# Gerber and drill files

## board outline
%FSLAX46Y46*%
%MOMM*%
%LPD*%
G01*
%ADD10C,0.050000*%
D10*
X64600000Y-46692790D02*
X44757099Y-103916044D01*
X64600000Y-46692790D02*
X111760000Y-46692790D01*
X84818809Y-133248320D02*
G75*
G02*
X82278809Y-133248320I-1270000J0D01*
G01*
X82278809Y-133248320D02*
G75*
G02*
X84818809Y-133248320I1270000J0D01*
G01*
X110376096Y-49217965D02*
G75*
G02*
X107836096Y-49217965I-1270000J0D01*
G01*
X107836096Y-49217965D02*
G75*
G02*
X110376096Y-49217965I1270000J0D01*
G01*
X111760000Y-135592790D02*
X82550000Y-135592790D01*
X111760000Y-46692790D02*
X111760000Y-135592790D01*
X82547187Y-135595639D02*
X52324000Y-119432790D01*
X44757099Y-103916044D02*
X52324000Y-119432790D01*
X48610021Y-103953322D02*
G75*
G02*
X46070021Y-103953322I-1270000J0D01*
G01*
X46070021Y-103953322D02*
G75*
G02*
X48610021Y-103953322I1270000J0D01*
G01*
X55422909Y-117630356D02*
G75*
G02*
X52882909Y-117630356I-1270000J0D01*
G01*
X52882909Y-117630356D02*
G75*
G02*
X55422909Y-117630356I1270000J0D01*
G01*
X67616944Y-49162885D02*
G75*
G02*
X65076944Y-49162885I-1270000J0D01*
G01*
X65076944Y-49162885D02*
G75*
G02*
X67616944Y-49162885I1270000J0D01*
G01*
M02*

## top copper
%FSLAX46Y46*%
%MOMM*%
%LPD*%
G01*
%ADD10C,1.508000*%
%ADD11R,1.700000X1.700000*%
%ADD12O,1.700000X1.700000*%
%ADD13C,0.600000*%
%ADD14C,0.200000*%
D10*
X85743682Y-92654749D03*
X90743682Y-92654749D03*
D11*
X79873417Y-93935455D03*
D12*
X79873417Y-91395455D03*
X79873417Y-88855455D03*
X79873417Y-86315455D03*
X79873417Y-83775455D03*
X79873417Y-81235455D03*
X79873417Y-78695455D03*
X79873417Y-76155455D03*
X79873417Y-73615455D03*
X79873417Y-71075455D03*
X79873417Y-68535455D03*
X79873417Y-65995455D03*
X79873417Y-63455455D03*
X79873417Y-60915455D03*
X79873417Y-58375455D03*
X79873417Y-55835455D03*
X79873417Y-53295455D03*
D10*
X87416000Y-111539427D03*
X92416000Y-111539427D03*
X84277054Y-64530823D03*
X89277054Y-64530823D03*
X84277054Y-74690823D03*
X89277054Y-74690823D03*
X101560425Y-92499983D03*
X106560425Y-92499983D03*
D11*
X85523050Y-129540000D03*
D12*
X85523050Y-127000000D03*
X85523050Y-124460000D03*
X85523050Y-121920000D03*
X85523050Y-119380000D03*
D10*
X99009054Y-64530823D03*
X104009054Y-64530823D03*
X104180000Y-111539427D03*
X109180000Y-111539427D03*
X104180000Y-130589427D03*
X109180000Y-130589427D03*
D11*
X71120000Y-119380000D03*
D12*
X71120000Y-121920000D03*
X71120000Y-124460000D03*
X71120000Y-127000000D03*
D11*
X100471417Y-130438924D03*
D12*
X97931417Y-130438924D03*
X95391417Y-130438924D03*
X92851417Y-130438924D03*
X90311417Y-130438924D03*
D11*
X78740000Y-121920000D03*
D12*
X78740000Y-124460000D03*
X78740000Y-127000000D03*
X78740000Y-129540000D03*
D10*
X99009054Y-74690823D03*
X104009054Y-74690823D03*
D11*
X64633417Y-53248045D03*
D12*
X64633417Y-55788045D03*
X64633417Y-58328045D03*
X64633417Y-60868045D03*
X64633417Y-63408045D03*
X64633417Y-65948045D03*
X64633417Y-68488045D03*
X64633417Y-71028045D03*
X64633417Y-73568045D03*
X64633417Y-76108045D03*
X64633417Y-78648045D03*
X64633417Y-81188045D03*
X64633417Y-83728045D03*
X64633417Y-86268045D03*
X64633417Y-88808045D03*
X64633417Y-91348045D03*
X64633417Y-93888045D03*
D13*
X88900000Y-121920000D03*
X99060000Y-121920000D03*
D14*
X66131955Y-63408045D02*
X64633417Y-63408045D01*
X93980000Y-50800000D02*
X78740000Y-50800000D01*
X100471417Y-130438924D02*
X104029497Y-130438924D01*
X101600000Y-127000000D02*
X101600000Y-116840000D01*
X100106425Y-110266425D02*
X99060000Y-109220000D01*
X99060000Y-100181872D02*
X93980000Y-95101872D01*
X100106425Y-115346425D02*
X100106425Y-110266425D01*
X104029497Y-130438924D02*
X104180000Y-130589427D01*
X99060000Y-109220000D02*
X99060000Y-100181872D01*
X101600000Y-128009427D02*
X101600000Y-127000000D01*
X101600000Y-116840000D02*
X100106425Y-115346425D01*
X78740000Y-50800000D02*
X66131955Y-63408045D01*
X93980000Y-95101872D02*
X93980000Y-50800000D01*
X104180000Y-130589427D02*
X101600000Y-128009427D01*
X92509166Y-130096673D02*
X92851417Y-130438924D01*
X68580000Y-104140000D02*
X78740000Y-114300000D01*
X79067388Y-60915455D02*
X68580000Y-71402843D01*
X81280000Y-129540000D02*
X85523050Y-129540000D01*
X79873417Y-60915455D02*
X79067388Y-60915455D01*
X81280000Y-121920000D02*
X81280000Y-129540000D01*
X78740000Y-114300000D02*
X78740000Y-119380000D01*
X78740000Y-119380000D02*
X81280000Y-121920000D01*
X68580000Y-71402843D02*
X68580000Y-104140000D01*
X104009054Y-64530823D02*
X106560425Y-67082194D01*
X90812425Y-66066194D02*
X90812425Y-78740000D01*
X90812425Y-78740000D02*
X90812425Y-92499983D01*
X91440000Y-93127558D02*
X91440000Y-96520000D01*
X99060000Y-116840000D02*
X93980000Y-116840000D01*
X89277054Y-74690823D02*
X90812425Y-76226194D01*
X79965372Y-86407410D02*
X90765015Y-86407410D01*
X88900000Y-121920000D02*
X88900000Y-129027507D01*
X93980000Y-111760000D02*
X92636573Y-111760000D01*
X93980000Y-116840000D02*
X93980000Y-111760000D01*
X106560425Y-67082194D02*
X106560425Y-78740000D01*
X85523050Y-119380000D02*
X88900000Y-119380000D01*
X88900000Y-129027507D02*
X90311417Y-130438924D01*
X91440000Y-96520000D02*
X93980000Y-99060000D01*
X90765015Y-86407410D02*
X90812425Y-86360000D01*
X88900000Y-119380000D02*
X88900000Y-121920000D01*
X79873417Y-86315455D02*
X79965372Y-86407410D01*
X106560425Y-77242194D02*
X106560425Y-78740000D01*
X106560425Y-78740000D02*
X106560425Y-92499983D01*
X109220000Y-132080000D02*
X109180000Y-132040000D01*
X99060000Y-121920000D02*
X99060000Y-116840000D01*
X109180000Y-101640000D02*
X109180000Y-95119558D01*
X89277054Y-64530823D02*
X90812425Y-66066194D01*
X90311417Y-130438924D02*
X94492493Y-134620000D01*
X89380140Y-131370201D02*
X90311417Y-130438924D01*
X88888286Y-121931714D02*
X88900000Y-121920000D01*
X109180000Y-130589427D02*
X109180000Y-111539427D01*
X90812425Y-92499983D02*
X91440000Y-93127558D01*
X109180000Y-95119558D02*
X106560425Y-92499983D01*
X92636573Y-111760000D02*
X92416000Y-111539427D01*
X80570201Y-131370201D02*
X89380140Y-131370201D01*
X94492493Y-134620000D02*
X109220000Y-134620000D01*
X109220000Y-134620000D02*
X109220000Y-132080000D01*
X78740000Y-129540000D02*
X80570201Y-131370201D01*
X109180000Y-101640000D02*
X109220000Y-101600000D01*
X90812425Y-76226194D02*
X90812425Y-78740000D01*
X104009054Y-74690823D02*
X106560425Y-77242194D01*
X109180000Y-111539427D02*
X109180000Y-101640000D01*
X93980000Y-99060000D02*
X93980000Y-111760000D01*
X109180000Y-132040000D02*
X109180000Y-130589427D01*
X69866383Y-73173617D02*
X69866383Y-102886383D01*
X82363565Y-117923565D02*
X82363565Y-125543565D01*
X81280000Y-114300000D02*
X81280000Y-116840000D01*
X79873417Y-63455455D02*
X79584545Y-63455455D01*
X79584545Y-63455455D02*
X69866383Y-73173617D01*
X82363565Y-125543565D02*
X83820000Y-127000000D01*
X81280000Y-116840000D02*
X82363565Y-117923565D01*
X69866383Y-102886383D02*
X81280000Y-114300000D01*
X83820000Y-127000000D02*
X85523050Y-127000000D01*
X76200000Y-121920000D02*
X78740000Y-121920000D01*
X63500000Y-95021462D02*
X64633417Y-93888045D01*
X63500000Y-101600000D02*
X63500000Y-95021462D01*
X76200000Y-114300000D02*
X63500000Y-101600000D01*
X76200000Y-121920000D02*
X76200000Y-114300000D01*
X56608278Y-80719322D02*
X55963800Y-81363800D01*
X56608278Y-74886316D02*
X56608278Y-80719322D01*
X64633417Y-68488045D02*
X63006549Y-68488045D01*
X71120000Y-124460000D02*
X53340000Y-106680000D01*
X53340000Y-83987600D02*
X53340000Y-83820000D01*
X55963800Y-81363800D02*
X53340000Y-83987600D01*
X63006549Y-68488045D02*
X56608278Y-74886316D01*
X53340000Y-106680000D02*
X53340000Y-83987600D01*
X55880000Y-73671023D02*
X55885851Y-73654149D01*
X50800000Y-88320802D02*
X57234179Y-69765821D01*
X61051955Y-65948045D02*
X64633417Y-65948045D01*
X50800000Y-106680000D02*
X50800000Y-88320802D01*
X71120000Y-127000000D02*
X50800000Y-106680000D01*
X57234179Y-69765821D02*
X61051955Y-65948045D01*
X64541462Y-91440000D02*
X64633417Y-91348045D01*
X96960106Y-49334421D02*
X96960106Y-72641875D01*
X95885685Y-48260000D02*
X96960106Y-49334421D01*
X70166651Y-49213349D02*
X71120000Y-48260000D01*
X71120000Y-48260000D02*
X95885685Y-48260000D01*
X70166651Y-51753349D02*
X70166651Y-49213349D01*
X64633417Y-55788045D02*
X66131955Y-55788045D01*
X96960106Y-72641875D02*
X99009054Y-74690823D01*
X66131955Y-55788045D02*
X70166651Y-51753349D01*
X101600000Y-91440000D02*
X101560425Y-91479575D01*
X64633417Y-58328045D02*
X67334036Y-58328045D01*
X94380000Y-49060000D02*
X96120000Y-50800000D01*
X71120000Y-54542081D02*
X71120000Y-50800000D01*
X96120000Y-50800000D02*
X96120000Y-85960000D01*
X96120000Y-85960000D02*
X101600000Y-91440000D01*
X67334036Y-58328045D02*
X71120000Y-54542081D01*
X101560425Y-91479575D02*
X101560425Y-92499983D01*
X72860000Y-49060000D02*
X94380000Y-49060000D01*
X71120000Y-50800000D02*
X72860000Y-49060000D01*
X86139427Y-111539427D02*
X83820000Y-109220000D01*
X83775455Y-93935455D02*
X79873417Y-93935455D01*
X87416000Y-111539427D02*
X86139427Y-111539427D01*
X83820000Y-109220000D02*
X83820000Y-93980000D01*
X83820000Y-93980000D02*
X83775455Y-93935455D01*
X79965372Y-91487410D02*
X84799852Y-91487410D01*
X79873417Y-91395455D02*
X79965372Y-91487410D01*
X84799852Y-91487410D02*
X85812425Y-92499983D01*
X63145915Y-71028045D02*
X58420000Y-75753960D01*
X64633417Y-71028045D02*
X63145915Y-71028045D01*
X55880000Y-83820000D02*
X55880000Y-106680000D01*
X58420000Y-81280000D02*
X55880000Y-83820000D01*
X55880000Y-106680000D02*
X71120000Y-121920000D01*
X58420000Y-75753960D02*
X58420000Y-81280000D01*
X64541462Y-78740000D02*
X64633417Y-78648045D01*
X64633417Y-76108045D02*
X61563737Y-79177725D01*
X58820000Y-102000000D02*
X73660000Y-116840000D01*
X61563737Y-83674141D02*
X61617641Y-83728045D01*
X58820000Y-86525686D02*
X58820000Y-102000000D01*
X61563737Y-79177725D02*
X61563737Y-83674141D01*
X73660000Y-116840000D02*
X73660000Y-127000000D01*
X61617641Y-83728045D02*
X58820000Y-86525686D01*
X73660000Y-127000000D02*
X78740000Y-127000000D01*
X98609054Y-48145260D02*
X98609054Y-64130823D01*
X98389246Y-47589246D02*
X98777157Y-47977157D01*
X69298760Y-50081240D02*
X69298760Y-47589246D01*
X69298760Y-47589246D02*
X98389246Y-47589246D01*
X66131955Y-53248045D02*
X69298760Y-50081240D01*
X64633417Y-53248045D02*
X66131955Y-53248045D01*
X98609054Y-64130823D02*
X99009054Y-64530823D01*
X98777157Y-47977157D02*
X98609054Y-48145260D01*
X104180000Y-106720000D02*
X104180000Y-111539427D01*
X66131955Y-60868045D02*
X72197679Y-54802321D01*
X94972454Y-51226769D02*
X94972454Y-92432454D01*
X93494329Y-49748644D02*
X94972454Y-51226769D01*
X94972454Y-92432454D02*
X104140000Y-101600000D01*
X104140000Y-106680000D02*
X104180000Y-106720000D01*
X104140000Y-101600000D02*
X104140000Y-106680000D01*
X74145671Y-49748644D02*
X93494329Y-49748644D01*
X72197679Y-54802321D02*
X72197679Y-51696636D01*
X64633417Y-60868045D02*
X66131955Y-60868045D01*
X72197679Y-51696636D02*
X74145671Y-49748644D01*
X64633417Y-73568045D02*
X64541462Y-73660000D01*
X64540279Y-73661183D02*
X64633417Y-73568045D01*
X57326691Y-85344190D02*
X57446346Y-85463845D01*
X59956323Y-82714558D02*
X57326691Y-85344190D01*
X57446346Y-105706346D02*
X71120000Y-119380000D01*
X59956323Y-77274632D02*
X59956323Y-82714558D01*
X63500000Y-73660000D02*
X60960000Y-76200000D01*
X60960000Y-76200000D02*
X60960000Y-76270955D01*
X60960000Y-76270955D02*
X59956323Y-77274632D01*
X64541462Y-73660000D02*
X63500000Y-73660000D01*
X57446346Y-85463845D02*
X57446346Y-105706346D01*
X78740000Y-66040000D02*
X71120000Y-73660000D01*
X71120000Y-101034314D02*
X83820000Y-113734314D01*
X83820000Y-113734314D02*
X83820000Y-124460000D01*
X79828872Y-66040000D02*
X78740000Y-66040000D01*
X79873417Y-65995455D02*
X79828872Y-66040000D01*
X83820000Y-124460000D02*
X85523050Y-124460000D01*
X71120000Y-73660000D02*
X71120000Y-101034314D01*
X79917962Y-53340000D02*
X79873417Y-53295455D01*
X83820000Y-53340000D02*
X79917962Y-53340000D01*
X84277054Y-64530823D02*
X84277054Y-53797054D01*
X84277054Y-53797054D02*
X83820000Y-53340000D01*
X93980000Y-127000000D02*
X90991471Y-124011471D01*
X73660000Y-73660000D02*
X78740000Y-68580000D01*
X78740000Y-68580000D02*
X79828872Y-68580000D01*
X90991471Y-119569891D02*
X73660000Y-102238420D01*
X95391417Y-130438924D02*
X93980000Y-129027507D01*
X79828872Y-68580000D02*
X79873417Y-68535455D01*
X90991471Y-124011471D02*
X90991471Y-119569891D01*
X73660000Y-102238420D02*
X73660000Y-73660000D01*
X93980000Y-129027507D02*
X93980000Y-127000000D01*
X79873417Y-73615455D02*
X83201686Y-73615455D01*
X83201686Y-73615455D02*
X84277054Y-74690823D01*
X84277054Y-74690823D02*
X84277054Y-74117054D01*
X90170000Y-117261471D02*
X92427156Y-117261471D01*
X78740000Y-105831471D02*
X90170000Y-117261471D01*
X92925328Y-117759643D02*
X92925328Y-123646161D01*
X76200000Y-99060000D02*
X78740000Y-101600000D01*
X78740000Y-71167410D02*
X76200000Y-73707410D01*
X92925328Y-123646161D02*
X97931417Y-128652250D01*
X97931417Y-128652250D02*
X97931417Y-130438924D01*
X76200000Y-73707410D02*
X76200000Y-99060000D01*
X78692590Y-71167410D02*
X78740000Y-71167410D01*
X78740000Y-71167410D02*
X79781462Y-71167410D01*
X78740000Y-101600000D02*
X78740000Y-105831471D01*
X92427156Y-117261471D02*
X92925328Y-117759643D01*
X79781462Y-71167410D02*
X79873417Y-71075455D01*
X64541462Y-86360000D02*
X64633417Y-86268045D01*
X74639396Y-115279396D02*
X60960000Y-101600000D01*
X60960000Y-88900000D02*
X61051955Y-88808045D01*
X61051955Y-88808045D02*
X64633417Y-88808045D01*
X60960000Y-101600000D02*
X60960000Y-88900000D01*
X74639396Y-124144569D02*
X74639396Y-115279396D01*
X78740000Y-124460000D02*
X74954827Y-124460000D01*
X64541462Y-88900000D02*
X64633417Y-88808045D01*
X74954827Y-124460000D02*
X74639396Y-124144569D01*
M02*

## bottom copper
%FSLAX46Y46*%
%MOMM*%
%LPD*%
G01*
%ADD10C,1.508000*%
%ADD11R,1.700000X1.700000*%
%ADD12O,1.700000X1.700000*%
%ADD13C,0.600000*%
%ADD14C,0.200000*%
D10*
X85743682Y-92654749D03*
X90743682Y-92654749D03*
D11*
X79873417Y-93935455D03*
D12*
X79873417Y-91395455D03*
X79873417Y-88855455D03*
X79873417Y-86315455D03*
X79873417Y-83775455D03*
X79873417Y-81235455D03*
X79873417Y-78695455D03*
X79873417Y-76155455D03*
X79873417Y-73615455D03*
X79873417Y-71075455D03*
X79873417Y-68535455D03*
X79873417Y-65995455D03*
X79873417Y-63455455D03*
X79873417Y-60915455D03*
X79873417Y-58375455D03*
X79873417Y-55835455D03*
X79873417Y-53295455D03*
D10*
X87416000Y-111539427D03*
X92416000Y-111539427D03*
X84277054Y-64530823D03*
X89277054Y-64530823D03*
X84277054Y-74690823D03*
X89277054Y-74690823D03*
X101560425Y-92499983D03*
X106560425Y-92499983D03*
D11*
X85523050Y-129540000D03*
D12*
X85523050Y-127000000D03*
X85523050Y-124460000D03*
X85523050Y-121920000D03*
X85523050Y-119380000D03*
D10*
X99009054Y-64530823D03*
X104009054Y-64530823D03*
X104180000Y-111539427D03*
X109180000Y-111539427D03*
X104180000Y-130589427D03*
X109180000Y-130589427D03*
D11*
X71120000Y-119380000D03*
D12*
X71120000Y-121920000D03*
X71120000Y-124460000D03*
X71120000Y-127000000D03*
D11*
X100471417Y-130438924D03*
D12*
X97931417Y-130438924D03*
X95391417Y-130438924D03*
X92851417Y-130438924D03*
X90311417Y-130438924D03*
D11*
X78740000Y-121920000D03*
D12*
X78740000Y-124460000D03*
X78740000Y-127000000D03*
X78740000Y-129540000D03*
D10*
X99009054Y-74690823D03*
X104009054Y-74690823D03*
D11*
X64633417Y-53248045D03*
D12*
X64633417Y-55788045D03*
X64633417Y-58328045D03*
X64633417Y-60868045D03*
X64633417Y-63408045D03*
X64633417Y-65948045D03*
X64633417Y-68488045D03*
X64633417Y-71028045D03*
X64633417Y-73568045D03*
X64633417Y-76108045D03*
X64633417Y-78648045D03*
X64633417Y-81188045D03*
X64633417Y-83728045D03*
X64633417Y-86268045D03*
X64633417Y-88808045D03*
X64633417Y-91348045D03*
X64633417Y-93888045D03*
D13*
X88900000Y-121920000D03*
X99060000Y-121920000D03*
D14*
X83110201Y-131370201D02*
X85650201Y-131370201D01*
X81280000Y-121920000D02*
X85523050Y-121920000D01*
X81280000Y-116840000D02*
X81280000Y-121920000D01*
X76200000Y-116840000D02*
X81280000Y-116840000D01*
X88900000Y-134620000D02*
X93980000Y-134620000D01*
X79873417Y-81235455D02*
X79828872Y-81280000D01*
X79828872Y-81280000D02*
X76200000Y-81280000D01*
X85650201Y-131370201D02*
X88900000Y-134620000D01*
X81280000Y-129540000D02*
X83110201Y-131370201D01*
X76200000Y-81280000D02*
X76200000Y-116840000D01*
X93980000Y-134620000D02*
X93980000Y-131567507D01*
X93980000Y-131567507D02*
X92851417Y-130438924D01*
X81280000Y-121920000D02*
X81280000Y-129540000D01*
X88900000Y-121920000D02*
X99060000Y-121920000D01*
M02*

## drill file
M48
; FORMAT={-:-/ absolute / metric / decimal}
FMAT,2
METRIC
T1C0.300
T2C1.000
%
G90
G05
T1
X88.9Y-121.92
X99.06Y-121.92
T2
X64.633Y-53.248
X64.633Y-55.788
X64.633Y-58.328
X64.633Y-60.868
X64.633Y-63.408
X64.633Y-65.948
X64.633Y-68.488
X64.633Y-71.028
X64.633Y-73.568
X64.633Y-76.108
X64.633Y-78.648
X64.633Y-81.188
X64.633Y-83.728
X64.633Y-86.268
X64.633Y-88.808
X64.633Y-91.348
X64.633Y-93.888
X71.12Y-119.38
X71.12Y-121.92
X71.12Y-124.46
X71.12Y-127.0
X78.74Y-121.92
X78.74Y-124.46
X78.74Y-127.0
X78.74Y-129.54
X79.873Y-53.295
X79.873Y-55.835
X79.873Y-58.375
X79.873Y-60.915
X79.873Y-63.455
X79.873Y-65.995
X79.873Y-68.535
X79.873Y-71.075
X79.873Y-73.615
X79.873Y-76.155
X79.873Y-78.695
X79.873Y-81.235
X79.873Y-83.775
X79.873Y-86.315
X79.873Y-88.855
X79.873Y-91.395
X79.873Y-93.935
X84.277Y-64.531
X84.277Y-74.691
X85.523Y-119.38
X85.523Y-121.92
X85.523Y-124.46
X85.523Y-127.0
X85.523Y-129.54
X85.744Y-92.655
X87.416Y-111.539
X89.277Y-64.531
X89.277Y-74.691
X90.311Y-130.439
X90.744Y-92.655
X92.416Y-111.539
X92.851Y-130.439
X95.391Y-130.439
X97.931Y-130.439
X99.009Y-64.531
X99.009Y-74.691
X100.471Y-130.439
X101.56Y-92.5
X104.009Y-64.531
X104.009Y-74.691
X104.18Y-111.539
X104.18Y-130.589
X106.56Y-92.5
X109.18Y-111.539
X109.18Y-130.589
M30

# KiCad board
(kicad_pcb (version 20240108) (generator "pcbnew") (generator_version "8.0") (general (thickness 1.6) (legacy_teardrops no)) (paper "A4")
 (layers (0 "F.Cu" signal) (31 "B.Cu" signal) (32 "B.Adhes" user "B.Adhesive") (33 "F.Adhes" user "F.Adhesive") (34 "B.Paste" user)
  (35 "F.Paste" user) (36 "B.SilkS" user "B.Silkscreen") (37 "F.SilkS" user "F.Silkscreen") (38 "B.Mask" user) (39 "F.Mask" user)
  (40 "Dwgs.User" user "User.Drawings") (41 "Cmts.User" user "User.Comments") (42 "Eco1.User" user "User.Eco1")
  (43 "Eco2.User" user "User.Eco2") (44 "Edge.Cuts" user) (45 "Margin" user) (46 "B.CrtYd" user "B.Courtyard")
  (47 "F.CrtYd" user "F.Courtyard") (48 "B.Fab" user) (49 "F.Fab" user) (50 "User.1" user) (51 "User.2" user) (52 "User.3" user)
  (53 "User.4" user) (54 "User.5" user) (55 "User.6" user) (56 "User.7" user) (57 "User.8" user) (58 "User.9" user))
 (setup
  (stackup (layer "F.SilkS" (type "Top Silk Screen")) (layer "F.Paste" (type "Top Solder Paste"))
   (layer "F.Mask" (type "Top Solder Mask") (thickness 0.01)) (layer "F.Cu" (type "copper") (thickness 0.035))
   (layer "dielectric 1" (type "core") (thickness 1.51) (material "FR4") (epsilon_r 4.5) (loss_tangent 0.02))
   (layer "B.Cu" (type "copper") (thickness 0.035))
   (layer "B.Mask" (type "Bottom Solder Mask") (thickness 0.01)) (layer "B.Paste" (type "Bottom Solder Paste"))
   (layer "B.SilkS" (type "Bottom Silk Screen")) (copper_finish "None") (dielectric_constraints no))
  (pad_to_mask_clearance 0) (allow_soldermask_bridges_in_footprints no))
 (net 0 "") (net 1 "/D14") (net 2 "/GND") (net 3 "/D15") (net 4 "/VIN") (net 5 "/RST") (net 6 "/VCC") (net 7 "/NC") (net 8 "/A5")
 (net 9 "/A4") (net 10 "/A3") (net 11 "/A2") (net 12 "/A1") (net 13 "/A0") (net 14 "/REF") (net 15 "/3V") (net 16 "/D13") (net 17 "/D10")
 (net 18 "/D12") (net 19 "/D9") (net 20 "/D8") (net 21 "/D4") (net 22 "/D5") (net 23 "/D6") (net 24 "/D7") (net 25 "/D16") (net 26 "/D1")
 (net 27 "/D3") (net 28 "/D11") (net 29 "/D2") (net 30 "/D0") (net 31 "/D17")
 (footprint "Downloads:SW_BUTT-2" (layer "F.Cu") (at 88.243682 92.654749)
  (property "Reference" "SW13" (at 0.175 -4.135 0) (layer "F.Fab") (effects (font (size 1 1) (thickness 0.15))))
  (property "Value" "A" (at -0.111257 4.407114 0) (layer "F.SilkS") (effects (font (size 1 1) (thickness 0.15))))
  (pad "1" thru_hole circle (at -2.5 0) (size 1.508 1.508) (drill 1) (layers "*.Cu" "*.Mask") (remove_unused_layers no) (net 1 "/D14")
   (solder_mask_margin 0.102))
  (pad "2" thru_hole circle (at 2.5 0) (size 1.508 1.508) (drill 1) (layers "*.Cu" "*.Mask") (remove_unused_layers no) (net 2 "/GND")
   (solder_mask_margin 0.102)))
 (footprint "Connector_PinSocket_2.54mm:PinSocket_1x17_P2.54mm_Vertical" (layer "F.Cu") (at 79.873417 93.935455 180)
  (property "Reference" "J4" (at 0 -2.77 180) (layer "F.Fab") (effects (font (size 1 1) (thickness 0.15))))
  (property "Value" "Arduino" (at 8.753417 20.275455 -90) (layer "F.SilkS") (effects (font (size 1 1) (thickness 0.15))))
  (pad "1" thru_hole rect (at 0 0 180) (size 1.7 1.7) (drill 1) (layers "*.Cu" "*.Mask") (remove_unused_layers no) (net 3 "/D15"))
  (pad "2" thru_hole oval (at 0 2.54 180) (size 1.7 1.7) (drill 1) (layers "*.Cu" "*.Mask") (remove_unused_layers no) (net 1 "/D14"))
  (pad "3" thru_hole oval (at 0 5.08 180) (size 1.7 1.7) (drill 1) (layers "*.Cu" "*.Mask") (remove_unused_layers no) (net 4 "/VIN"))
  (pad "4" thru_hole oval (at 0 7.62 180) (size 1.7 1.7) (drill 1) (layers "*.Cu" "*.Mask") (remove_unused_layers no) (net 2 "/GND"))
  (pad "5" thru_hole oval (at 0 10.16 180) (size 1.7 1.7) (drill 1) (layers "*.Cu" "*.Mask") (remove_unused_layers no) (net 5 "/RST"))
  (pad "6" thru_hole oval (at 0 12.7 180) (size 1.7 1.7) (drill 1) (layers "*.Cu" "*.Mask") (remove_unused_layers no) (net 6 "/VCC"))
  (pad "7" thru_hole oval (at 0 15.24 180) (size 1.7 1.7) (drill 1) (layers "*.Cu" "*.Mask") (remove_unused_layers no) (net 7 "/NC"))
  (pad "8" thru_hole oval (at 0 17.78 180) (size 1.7 1.7) (drill 1) (layers "*.Cu" "*.Mask") (remove_unused_layers no) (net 7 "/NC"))
  (pad "9" thru_hole oval (at 0 20.32 180) (size 1.7 1.7) (drill 1) (layers "*.Cu" "*.Mask") (remove_unused_layers no) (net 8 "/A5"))
  (pad "10" thru_hole oval (at 0 22.86 180) (size 1.7 1.7) (drill 1) (layers "*.Cu" "*.Mask") (remove_unused_layers no) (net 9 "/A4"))
  (pad "11" thru_hole oval (at 0 25.4 180) (size 1.7 1.7) (drill 1) (layers "*.Cu" "*.Mask") (remove_unused_layers no) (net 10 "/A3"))
  (pad "12" thru_hole oval (at 0 27.94 180) (size 1.7 1.7) (drill 1) (layers "*.Cu" "*.Mask") (remove_unused_layers no) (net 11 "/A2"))
  (pad "13" thru_hole oval (at 0 30.48 180) (size 1.7 1.7) (drill 1) (layers "*.Cu" "*.Mask") (remove_unused_layers no) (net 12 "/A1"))
  (pad "14" thru_hole oval (at 0 33.02 180) (size 1.7 1.7) (drill 1) (layers "*.Cu" "*.Mask") (remove_unused_layers no) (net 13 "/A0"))
  (pad "15" thru_hole oval (at 0 35.56 180) (size 1.7 1.7) (drill 1) (layers "*.Cu" "*.Mask") (remove_unused_layers no) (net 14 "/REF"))
  (pad "16" thru_hole oval (at 0 38.1 180) (size 1.7 1.7) (drill 1) (layers "*.Cu" "*.Mask") (remove_unused_layers no) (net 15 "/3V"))
  (pad "17" thru_hole oval (at 0 40.64 180) (size 1.7 1.7) (drill 1) (layers "*.Cu" "*.Mask") (remove_unused_layers no) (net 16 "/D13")))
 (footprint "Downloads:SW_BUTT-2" (layer "F.Cu") (at 89.916 111.539427)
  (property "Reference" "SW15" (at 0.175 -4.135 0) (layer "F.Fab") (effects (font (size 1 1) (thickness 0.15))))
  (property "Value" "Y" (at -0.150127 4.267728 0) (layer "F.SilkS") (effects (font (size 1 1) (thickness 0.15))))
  (pad "1" thru_hole circle (at -2.5 0) (size 1.508 1.508) (drill 1) (layers "*.Cu" "*.Mask") (remove_unused_layers no) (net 3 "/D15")
   (solder_mask_margin 0.102))
  (pad "2" thru_hole circle (at 2.5 0) (size 1.508 1.508) (drill 1) (layers "*.Cu" "*.Mask") (remove_unused_layers no) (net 2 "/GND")
   (solder_mask_margin 0.102)))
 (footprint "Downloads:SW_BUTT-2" (layer "F.Cu") (at 86.777054 64.530823)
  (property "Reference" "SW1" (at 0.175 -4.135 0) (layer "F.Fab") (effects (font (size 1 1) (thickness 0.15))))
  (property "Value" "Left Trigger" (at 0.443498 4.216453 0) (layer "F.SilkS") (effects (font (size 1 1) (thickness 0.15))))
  (pad "1" thru_hole circle (at -2.5 0) (size 1.508 1.508) (drill 1) (layers "*.Cu" "*.Mask") (remove_unused_layers no) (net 16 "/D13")
   (solder_mask_margin 0.102))
  (pad "2" thru_hole circle (at 2.5 0) (size 1.508 1.508) (drill 1) (layers "*.Cu" "*.Mask") (remove_unused_layers no) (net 2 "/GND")
   (solder_mask_margin 0.102)))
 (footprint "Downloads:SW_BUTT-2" (layer "F.Cu") (at 86.777054 74.690823)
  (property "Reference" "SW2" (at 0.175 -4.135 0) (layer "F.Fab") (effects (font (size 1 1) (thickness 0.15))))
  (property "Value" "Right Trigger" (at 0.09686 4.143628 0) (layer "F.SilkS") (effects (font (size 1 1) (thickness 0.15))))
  (pad "1" thru_hole circle (at -2.5 0) (size 1.508 1.508) (drill 1) (layers "*.Cu" "*.Mask") (remove_unused_layers no) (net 8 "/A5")
   (solder_mask_margin 0.102))
  (pad "2" thru_hole circle (at 2.5 0) (size 1.508 1.508) (drill 1) (layers "*.Cu" "*.Mask") (remove_unused_layers no) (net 2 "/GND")
   (solder_mask_margin 0.102)))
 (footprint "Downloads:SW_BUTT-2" (layer "F.Cu") (at 104.060425 92.499983)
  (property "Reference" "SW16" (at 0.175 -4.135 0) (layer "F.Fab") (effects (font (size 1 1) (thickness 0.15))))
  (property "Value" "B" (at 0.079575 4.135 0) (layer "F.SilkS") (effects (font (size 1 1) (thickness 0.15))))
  (pad "1" thru_hole circle (at -2.5 0) (size 1.508 1.508) (drill 1) (layers "*.Cu" "*.Mask") (remove_unused_layers no) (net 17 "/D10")
   (solder_mask_margin 0.102))
  (pad "2" thru_hole circle (at 2.5 0) (size 1.508 1.508) (drill 1) (layers "*.Cu" "*.Mask") (remove_unused_layers no) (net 2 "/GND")
   (solder_mask_margin 0.102)))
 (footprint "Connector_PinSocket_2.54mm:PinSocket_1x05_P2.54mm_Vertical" (layer "F.Cu") (at 85.52305 129.54 180)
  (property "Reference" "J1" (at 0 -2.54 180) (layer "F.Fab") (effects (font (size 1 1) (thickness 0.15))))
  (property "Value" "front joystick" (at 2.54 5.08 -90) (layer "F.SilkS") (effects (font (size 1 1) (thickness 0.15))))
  (pad "1" thru_hole rect (at 0 0 180) (size 1.7 1.7) (drill 1) (layers "*.Cu" "*.Mask") (remove_unused_layers no) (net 13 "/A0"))
  (pad "2" thru_hole oval (at 0 2.54 180) (size 1.7 1.7) (drill 1) (layers "*.Cu" "*.Mask") (remove_unused_layers no) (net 12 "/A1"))
  (pad "3" thru_hole oval (at 0 5.08 180) (size 1.7 1.7) (drill 1) (layers "*.Cu" "*.Mask") (remove_unused_layers no) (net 11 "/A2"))
  (pad "4" thru_hole oval (at 0 7.62 180) (size 1.7 1.7) (drill 1) (layers "*.Cu" "*.Mask") (remove_unused_layers no) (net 6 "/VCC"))
  (pad "5" thru_hole oval (at 0 10.16 180) (size 1.7 1.7) (drill 1) (layers "*.Cu" "*.Mask") (remove_unused_layers no) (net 2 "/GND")))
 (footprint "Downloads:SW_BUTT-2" (layer "F.Cu") (at 101.509054 64.530823)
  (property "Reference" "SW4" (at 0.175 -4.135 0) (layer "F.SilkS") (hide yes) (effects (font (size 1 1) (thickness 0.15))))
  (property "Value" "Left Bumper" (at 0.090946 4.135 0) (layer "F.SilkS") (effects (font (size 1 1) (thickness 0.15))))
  (pad "1" thru_hole circle (at -2.5 0) (size 1.508 1.508) (drill 1) (layers "*.Cu" "*.Mask") (remove_unused_layers no) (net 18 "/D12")
   (solder_mask_margin 0.102))
  (pad "2" thru_hole circle (at 2.5 0) (size 1.508 1.508) (drill 1) (layers "*.Cu" "*.Mask") (remove_unused_layers no) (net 2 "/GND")
   (solder_mask_margin 0.102)))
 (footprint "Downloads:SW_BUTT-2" (layer "F.Cu") (at 106.68 111.539427)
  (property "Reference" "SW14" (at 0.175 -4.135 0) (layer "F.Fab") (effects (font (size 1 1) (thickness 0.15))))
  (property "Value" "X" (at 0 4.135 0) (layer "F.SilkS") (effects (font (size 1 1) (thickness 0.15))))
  (pad "1" thru_hole circle (at -2.5 0) (size 1.508 1.508) (drill 1) (layers "*.Cu" "*.Mask") (remove_unused_layers no) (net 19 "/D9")
   (solder_mask_margin 0.102))
  (pad "2" thru_hole circle (at 2.5 0) (size 1.508 1.508) (drill 1) (layers "*.Cu" "*.Mask") (remove_unused_layers no) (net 2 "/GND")
   (solder_mask_margin 0.102)))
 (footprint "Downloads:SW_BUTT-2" (layer "F.Cu") (at 106.68 130.589427)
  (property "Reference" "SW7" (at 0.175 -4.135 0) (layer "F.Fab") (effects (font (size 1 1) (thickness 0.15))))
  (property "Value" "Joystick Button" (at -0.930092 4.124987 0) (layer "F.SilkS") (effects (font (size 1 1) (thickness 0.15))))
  (pad "1" thru_hole circle (at -2.5 0) (size 1.508 1.508) (drill 1) (layers "*.Cu" "*.Mask") (remove_unused_layers no) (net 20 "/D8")
   (solder_mask_margin 0.102))
  (pad "2" thru_hole circle (at 2.5 0) (size 1.508 1.508) (drill 1) (layers "*.Cu" "*.Mask") (remove_unused_layers no) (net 2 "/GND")
   (solder_mask_margin 0.102)))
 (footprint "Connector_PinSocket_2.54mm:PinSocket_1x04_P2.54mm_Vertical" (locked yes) (layer "F.Cu") (at 71.12 119.38)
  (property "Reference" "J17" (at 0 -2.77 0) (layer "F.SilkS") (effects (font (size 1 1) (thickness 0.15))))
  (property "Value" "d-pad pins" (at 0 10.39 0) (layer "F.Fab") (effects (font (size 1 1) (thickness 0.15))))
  (pad "1" thru_hole rect (at 0 0) (size 1.7 1.7) (drill 1) (layers "*.Cu" "*.Mask") (remove_unused_layers no) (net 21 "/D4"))
  (pad "2" thru_hole oval (at 0 2.54) (size 1.7 1.7) (drill 1) (layers "*.Cu" "*.Mask") (remove_unused_layers no) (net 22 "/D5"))
  (pad "3" thru_hole oval (at 0 5.08) (size 1.7 1.7) (drill 1) (layers "*.Cu" "*.Mask") (remove_unused_layers no) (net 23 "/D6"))
  (pad "4" thru_hole oval (at 0 7.62) (size 1.7 1.7) (drill 1) (layers "*.Cu" "*.Mask") (remove_unused_layers no) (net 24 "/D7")))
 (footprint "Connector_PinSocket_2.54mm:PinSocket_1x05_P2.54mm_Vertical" (layer "F.Cu") (at 100.471417 130.438924 -90)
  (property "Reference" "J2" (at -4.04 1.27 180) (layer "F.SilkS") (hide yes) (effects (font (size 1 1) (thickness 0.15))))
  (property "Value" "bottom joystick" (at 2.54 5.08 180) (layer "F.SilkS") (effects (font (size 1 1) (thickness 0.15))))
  (pad "1" thru_hole rect (at 0 0 270) (size 1.7 1.7) (drill 1) (layers "*.Cu" "*.Mask") (remove_unused_layers no) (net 20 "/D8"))
  (pad "2" thru_hole oval (at 0 2.54 270) (size 1.7 1.7) (drill 1) (layers "*.Cu" "*.Mask") (remove_unused_layers no) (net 9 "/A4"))
  (pad "3" thru_hole oval (at 0 5.08 270) (size 1.7 1.7) (drill 1) (layers "*.Cu" "*.Mask") (remove_unused_layers no) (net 10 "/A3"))
  (pad "4" thru_hole oval (at 0 7.62 270) (size 1.7 1.7) (drill 1) (layers "*.Cu" "*.Mask") (remove_unused_layers no) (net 6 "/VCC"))
  (pad "5" thru_hole oval (at 0 10.16 270) (size 1.7 1.7) (drill 1) (layers "*.Cu" "*.Mask") (remove_unused_layers no) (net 2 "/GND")))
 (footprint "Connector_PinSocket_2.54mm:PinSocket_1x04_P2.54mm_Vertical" (layer "F.Cu") (at 78.74 121.92)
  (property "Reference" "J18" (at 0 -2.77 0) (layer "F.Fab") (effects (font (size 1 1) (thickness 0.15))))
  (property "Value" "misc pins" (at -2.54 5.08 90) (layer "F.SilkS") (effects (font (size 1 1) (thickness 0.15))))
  (pad "1" thru_hole rect (at 0 0) (size 1.7 1.7) (drill 1) (layers "*.Cu" "*.Mask") (remove_unused_layers no) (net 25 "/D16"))
  (pad "2" thru_hole oval (at 0 2.54) (size 1.7 1.7) (drill 1) (layers "*.Cu" "*.Mask") (remove_unused_layers no) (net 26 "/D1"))
  (pad "3" thru_hole oval (at 0 5.08) (size 1.7 1.7) (drill 1) (layers "*.Cu" "*.Mask") (remove_unused_layers no) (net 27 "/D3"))
  (pad "4" thru_hole oval (at 0 7.62) (size 1.7 1.7) (drill 1) (layers "*.Cu" "*.Mask") (remove_unused_layers no) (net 2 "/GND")))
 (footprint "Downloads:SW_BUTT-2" (layer "F.Cu") (at 101.509054 74.690823)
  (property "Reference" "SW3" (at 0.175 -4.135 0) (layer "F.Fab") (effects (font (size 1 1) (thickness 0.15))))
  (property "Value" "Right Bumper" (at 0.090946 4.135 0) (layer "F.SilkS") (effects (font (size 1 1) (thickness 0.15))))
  (pad "1" thru_hole circle (at -2.5 0) (size 1.508 1.508) (drill 1) (layers "*.Cu" "*.Mask") (remove_unused_layers no) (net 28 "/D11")
   (solder_mask_margin 0.102))
  (pad "2" thru_hole circle (at 2.5 0) (size 1.508 1.508) (drill 1) (layers "*.Cu" "*.Mask") (remove_unused_layers no) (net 2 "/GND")
   (solder_mask_margin 0.102)))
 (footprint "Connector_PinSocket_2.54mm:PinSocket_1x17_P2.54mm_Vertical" (layer "F.Cu") (at 64.633417 53.248045)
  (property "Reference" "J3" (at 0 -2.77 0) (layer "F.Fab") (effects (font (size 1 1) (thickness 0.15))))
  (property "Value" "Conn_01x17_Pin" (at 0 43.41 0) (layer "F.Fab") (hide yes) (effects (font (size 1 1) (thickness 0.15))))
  (pad "1" thru_hole rect (at 0 0) (size 1.7 1.7) (drill 1) (layers "*.Cu" "*.Mask") (remove_unused_layers no) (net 18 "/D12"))
  (pad "2" thru_hole oval (at 0 2.54) (size 1.7 1.7) (drill 1) (layers "*.Cu" "*.Mask") (remove_unused_layers no) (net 28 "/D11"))
  (pad "3" thru_hole oval (at 0 5.08) (size 1.7 1.7) (drill 1) (layers "*.Cu" "*.Mask") (remove_unused_layers no) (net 17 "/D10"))
  (pad "4" thru_hole oval (at 0 7.62) (size 1.7 1.7) (drill 1) (layers "*.Cu" "*.Mask") (remove_unused_layers no) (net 19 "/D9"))
  (pad "5" thru_hole oval (at 0 10.16) (size 1.7 1.7) (drill 1) (layers "*.Cu" "*.Mask") (remove_unused_layers no) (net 20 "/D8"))
  (pad "6" thru_hole oval (at 0 12.7) (size 1.7 1.7) (drill 1) (layers "*.Cu" "*.Mask") (remove_unused_layers no) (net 24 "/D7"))
  (pad "7" thru_hole oval (at 0 15.24) (size 1.7 1.7) (drill 1) (layers "*.Cu" "*.Mask") (remove_unused_layers no) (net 23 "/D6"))
  (pad "8" thru_hole oval (at 0 17.78) (size 1.7 1.7) (drill 1) (layers "*.Cu" "*.Mask") (remove_unused_layers no) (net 22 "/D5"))
  (pad "9" thru_hole oval (at 0 20.32) (size 1.7 1.7) (drill 1) (layers "*.Cu" "*.Mask") (remove_unused_layers no) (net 21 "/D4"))
  (pad "10" thru_hole oval (at 0 22.86) (size 1.7 1.7) (drill 1) (layers "*.Cu" "*.Mask") (remove_unused_layers no) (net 27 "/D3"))
  (pad "11" thru_hole oval (at 0 25.4) (size 1.7 1.7) (drill 1) (layers "*.Cu" "*.Mask") (remove_unused_layers no) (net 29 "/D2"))
  (pad "12" thru_hole oval (at 0 27.94) (size 1.7 1.7) (drill 1) (layers "*.Cu" "*.Mask") (remove_unused_layers no) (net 2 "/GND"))
  (pad "13" thru_hole oval (at 0 30.48) (size 1.7 1.7) (drill 1) (layers "*.Cu" "*.Mask") (remove_unused_layers no) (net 5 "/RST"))
  (pad "14" thru_hole oval (at 0 33.02) (size 1.7 1.7) (drill 1) (layers "*.Cu" "*.Mask") (remove_unused_layers no) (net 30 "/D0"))
  (pad "15" thru_hole oval (at 0 35.56) (size 1.7 1.7) (drill 1) (layers "*.Cu" "*.Mask") (remove_unused_layers no) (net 26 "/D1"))
  (pad "16" thru_hole oval (at 0 38.1) (size 1.7 1.7) (drill 1) (layers "*.Cu" "*.Mask") (remove_unused_layers no) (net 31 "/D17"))
  (pad "17" thru_hole oval (at 0 40.64) (size 1.7 1.7) (drill 1) (layers "*.Cu" "*.Mask") (remove_unused_layers no) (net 25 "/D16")))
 (gr_line (start 64.6 46.69279) (end 44.757099 103.916044) (stroke (width 0.05) (type default)) (layer "Edge.Cuts"))
 (gr_line (start 64.6 46.69279) (end 111.76 46.69279) (stroke (width 0.05) (type default)) (layer "Edge.Cuts"))
 (gr_circle (center 83.548809 133.24832) (end 82.278809 133.24832) (stroke (width 0.05) (type default)) (fill none) (layer "Edge.Cuts"))
 (gr_circle (center 109.106096 49.217965) (end 110.376096 49.217965) (stroke (width 0.05) (type default)) (fill none) (layer "Edge.Cuts"))
 (gr_line (start 111.76 135.59279) (end 82.55 135.59279) (stroke (width 0.05) (type default)) (layer "Edge.Cuts"))
 (gr_line (start 111.76 46.69279) (end 111.76 135.59279) (stroke (width 0.05) (type default)) (layer "Edge.Cuts"))
 (gr_line (start 82.547187 135.595639) (end 52.324 119.43279) (stroke (width 0.05) (type default)) (layer "Edge.Cuts"))
 (gr_line (start 44.757099 103.916044) (end 52.324 119.43279) (stroke (width 0.05) (type default)) (layer "Edge.Cuts"))
 (gr_circle (center 47.340021 103.953322) (end 46.070021 103.953322) (stroke (width 0.05) (type default)) (fill none) (layer "Edge.Cuts"))
 (gr_circle (center 54.152909 117.630356) (end 52.882909 117.630356) (stroke (width 0.05) (type default)) (fill none) (layer "Edge.Cuts"))
 (gr_circle (center 66.346944 49.162885) (end 66.346944 47.892885) (stroke (width 0.05) (type default)) (fill none) (layer "Edge.Cuts"))
 (segment (start 66.131955 63.408045) (end 64.633417 63.408045) (width 0.2) (layer "F.Cu") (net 20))
 (segment (start 93.98 50.8) (end 78.74 50.8) (width 0.2) (layer "F.Cu") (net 20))
 (segment (start 100.471417 130.438924) (end 104.029497 130.438924) (width 0.2) (layer "F.Cu") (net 20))
 (segment (start 101.6 127) (end 101.6 116.84) (width 0.2) (layer "F.Cu") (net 20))
 (segment (start 100.106425 110.266425) (end 99.06 109.22) (width 0.2) (layer "F.Cu") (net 20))
 (segment (start 99.06 100.181872) (end 93.98 95.101872) (width 0.2) (layer "F.Cu") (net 20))
 (segment (start 100.106425 115.346425) (end 100.106425 110.266425) (width 0.2) (layer "F.Cu") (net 20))
 (segment (start 104.029497 130.438924) (end 104.18 130.589427) (width 0.2) (layer "F.Cu") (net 20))
 (segment (start 99.06 109.22) (end 99.06 100.181872) (width 0.2) (layer "F.Cu") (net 20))
 (segment (start 101.6 128.009427) (end 101.6 127) (width 0.2) (layer "F.Cu") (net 20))
 (segment (start 101.6 116.84) (end 100.106425 115.346425) (width 0.2) (layer "F.Cu") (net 20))
 (segment (start 78.74 50.8) (end 66.131955 63.408045) (width 0.2) (layer "F.Cu") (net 20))
 (segment (start 93.98 95.101872) (end 93.98 50.8) (width 0.2) (layer "F.Cu") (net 20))
 (segment (start 104.18 130.589427) (end 101.6 128.009427) (width 0.2) (layer "F.Cu") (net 20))
 (segment (start 92.509166 130.096673) (end 92.851417 130.438924) (width 0.2) (layer "F.Cu") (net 6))
 (segment (start 83.110201 131.370201) (end 85.650201 131.370201) (width 0.2) (layer "B.Cu") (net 6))
 (segment (start 81.28 121.92) (end 85.52305 121.92) (width 0.2) (layer "B.Cu") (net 6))
 (segment (start 81.28 116.84) (end 81.28 121.92) (width 0.2) (layer "B.Cu") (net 6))
 (segment (start 76.2 116.84) (end 81.28 116.84) (width 0.2) (layer "B.Cu") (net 6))
 (segment (start 88.9 134.62) (end 93.98 134.62) (width 0.2) (layer "B.Cu") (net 6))
 (segment (start 79.873417 81.235455) (end 79.828872 81.28) (width 0.2) (layer "B.Cu") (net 6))
 (segment (start 79.828872 81.28) (end 76.2 81.28) (width 0.2) (layer "B.Cu") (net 6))
 (segment (start 85.650201 131.370201) (end 88.9 134.62) (width 0.2) (layer "B.Cu") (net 6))
 (segment (start 81.28 129.54) (end 83.110201 131.370201) (width 0.2) (layer "B.Cu") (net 6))
 (segment (start 76.2 81.28) (end 76.2 116.84) (width 0.2) (layer "B.Cu") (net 6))
 (segment (start 93.98 134.62) (end 93.98 131.567507) (width 0.2) (layer "B.Cu") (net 6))
 (segment (start 93.98 131.567507) (end 92.851417 130.438924) (width 0.2) (layer "B.Cu") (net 6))
 (segment (start 81.28 121.92) (end 81.28 129.54) (width 0.2) (layer "B.Cu") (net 6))
 (segment (start 68.58 104.14) (end 78.74 114.3) (width 0.2) (layer "F.Cu") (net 13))
 (segment (start 79.067388 60.915455) (end 68.58 71.402843) (width 0.2) (layer "F.Cu") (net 13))
 (segment (start 81.28 129.54) (end 85.52305 129.54) (width 0.2) (layer "F.Cu") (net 13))
 (segment (start 79.873417 60.915455) (end 79.067388 60.915455) (width 0.2) (layer "F.Cu") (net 13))
 (segment (start 81.28 121.92) (end 81.28 129.54) (width 0.2) (layer "F.Cu") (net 13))
 (segment (start 78.74 114.3) (end 78.74 119.38) (width 0.2) (layer "F.Cu") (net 13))
 (segment (start 78.74 119.38) (end 81.28 121.92) (width 0.2) (layer "F.Cu") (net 13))
 (segment (start 68.58 71.402843) (end 68.58 104.14) (width 0.2) (layer "F.Cu") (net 13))
 (segment (start 104.009054 64.530823) (end 106.560425 67.082194) (width 0.2) (layer "F.Cu") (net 2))
 (segment (start 90.812425 66.066194) (end 90.812425 78.74) (width 0.2) (layer "F.Cu") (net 2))
 (segment (start 90.812425 78.74) (end 90.812425 92.499983) (width 0.2) (layer "F.Cu") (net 2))
 (segment (start 91.44 93.127558) (end 91.44 96.52) (width 0.2) (layer "F.Cu") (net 2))
 (segment (start 99.06 116.84) (end 93.98 116.84) (width 0.2) (layer "F.Cu") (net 2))
 (segment (start 89.277054 74.690823) (end 90.812425 76.226194) (width 0.2) (layer "F.Cu") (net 2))
 (segment (start 79.965372 86.40741) (end 90.765015 86.40741) (width 0.2) (layer "F.Cu") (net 2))
 (segment (start 88.9 121.92) (end 88.9 129.027507) (width 0.2) (layer "F.Cu") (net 2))
 (segment (start 93.98 111.76) (end 92.636573 111.76) (width 0.2) (layer "F.Cu") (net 2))
 (segment (start 93.98 116.84) (end 93.98 111.76) (width 0.2) (layer "F.Cu") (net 2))
 (segment (start 106.560425 67.082194) (end 106.560425 78.74) (width 0.2) (layer "F.Cu") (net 2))
 (segment (start 85.52305 119.38) (end 88.9 119.38) (width 0.2) (layer "F.Cu") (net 2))
 (segment (start 88.9 129.027507) (end 90.311417 130.438924) (width 0.2) (layer "F.Cu") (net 2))
 (segment (start 91.44 96.52) (end 93.98 99.06) (width 0.2) (layer "F.Cu") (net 2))
 (segment (start 90.765015 86.40741) (end 90.812425 86.36) (width 0.2) (layer "F.Cu") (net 2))
 (segment (start 88.9 119.38) (end 88.9 121.92) (width 0.2) (layer "F.Cu") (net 2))
 (segment (start 79.873417 86.315455) (end 79.965372 86.40741) (width 0.2) (layer "F.Cu") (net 2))
 (segment (start 106.560425 77.242194) (end 106.560425 78.74) (width 0.2) (layer "F.Cu") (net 2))
 (segment (start 106.560425 78.74) (end 106.560425 92.499983) (width 0.2) (layer "F.Cu") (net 2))
 (segment (start 109.22 132.08) (end 109.18 132.04) (width 0.2) (layer "F.Cu") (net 2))
 (segment (start 99.06 121.92) (end 99.06 116.84) (width 0.2) (layer "F.Cu") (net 2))
 (segment (start 109.18 101.64) (end 109.18 95.119558) (width 0.2) (layer "F.Cu") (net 2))
 (segment (start 89.277054 64.530823) (end 90.812425 66.066194) (width 0.2) (layer "F.Cu") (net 2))
 (segment (start 90.311417 130.438924) (end 94.492493 134.62) (width 0.2) (layer "F.Cu") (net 2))
 (segment (start 89.38014 131.370201) (end 90.311417 130.438924) (width 0.2) (layer "F.Cu") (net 2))
 (segment (start 88.888286 121.931714) (end 88.9 121.92) (width 0.2) (layer "F.Cu") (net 2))
 (segment (start 109.18 130.589427) (end 109.18 111.539427) (width 0.2) (layer "F.Cu") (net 2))
 (segment (start 90.812425 92.499983) (end 91.44 93.127558) (width 0.2) (layer "F.Cu") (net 2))
 (segment (start 109.18 95.119558) (end 106.560425 92.499983) (width 0.2) (layer "F.Cu") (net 2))
 (segment (start 92.636573 111.76) (end 92.416 111.539427) (width 0.2) (layer "F.Cu") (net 2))
 (segment (start 80.570201 131.370201) (end 89.38014 131.370201) (width 0.2) (layer "F.Cu") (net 2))
 (segment (start 94.492493 134.62) (end 109.22 134.62) (width 0.2) (layer "F.Cu") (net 2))
 (segment (start 109.22 134.62) (end 109.22 132.08) (width 0.2) (layer "F.Cu") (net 2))
 (segment (start 78.74 129.54) (end 80.570201 131.370201) (width 0.2) (layer "F.Cu") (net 2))
 (segment (start 109.18 101.64) (end 109.22 101.6) (width 0.2) (layer "F.Cu") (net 2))
 (segment (start 90.812425 76.226194) (end 90.812425 78.74) (width 0.2) (layer "F.Cu") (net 2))
 (segment (start 104.009054 74.690823) (end 106.560425 77.242194) (width 0.2) (layer "F.Cu") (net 2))
 (segment (start 109.18 111.539427) (end 109.18 101.64) (width 0.2) (layer "F.Cu") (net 2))
 (segment (start 93.98 99.06) (end 93.98 111.76) (width 0.2) (layer "F.Cu") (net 2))
 (segment (start 109.18 132.04) (end 109.18 130.589427) (width 0.2) (layer "F.Cu") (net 2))
 (via (at 88.9 121.92) (size 0.6) (drill 0.3) (layers "F.Cu" "B.Cu") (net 2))
 (via (at 99.06 121.92) (size 0.6) (drill 0.3) (layers "F.Cu" "B.Cu") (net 2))
 (segment (start 88.9 121.92) (end 99.06 121.92) (width 0.2) (layer "B.Cu") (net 2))
 (segment (start 69.866383 73.173617) (end 69.866383 102.886383) (width 0.2) (layer "F.Cu") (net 12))
 (segment (start 82.363565 117.923565) (end 82.363565 125.543565) (width 0.2) (layer "F.Cu") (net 12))
 (segment (start 81.28 114.3) (end 81.28 116.84) (width 0.2) (layer "F.Cu") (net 12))
 (segment (start 79.873417 63.455455) (end 79.584545 63.455455) (width 0.2) (layer "F.Cu") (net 12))
 (segment (start 79.584545 63.455455) (end 69.866383 73.173617) (width 0.2) (layer "F.Cu") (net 12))
 (segment (start 82.363565 125.543565) (end 83.82 127) (width 0.2) (layer "F.Cu") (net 12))
 (segment (start 81.28 116.84) (end 82.363565 117.923565) (width 0.2) (layer "F.Cu") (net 12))
 (segment (start 69.866383 102.886383) (end 81.28 114.3) (width 0.2) (layer "F.Cu") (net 12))
 (segment (start 83.82 127) (end 85.52305 127) (width 0.2) (layer "F.Cu") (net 12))
 (segment (start 76.2 121.92) (end 78.74 121.92) (width 0.2) (layer "F.Cu") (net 25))
 (segment (start 63.5 95.021462) (end 64.633417 93.888045) (width 0.2) (layer "F.Cu") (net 25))
 (segment (start 63.5 101.6) (end 63.5 95.021462) (width 0.2) (layer "F.Cu") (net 25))
 (segment (start 76.2 114.3) (end 63.5 101.6) (width 0.2) (layer "F.Cu") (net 25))
 (segment (start 76.2 121.92) (end 76.2 114.3) (width 0.2) (layer "F.Cu") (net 25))
 (segment (start 56.608278 80.719322) (end 55.9638 81.3638) (width 0.2) (layer "F.Cu") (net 23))
 (segment (start 56.608278 74.886316) (end 56.608278 80.719322) (width 0.2) (layer "F.Cu") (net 23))
 (segment (start 64.633417 68.488045) (end 63.006549 68.488045) (width 0.2) (layer "F.Cu") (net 23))
 (segment (start 71.12 124.46) (end 53.34 106.68) (width 0.2) (layer "F.Cu") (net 23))
 (segment (start 53.34 83.9876) (end 53.34 83.82) (width 0.2) (layer "F.Cu") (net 23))
 (segment (start 55.9638 81.3638) (end 53.34 83.9876) (width 0.2) (layer "F.Cu") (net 23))
 (segment (start 63.006549 68.488045) (end 56.608278 74.886316) (width 0.2) (layer "F.Cu") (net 23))
 (segment (start 53.34 106.68) (end 53.34 83.9876) (width 0.2) (layer "F.Cu") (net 23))
 (segment (start 55.88 73.671023) (end 55.885851 73.654149) (width 0.2) (layer "F.Cu") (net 24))
 (segment (start 50.8 88.320802) (end 57.234179 69.765821) (width 0.2) (layer "F.Cu") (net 24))
 (segment (start 61.051955 65.948045) (end 64.633417 65.948045) (width 0.2) (layer "F.Cu") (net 24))
 (segment (start 50.8 106.68) (end 50.8 88.320802) (width 0.2) (layer "F.Cu") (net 24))
 (segment (start 71.12 127) (end 50.8 106.68) (width 0.2) (layer "F.Cu") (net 24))
 (segment (start 57.234179 69.765821) (end 61.051955 65.948045) (width 0.2) (layer "F.Cu") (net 24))
 (segment (start 64.541462 91.44) (end 64.633417 91.348045) (width 0.2) (layer "F.Cu") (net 31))
 (segment (start 96.960106 49.334421) (end 96.960106 72.641875) (width 0.2) (layer "F.Cu") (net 28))
 (segment (start 95.885685 48.26) (end 96.960106 49.334421) (width 0.2) (layer "F.Cu") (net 28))
 (segment (start 70.166651 49.213349) (end 71.12 48.26) (width 0.2) (layer "F.Cu") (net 28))
 (segment (start 71.12 48.26) (end 95.885685 48.26) (width 0.2) (layer "F.Cu") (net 28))
 (segment (start 70.166651 51.753349) (end 70.166651 49.213349) (width 0.2) (layer "F.Cu") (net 28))
 (segment (start 64.633417 55.788045) (end 66.131955 55.788045) (width 0.2) (layer "F.Cu") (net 28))
 (segment (start 96.960106 72.641875) (end 99.009054 74.690823) (width 0.2) (layer "F.Cu") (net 28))
 (segment (start 66.131955 55.788045) (end 70.166651 51.753349) (width 0.2) (layer "F.Cu") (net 28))
 (segment (start 101.6 91.44) (end 101.560425 91.479575) (width 0.2) (layer "F.Cu") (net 17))
 (segment (start 64.633417 58.328045) (end 67.334036 58.328045) (width 0.2) (layer "F.Cu") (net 17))
 (segment (start 94.38 49.06) (end 96.12 50.8) (width 0.2) (layer "F.Cu") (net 17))
 (segment (start 71.12 54.542081) (end 71.12 50.8) (width 0.2) (layer "F.Cu") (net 17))
 (segment (start 96.12 50.8) (end 96.12 85.96) (width 0.2) (layer "F.Cu") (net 17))
 (segment (start 96.12 85.96) (end 101.6 91.44) (width 0.2) (layer "F.Cu") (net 17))
 (segment (start 67.334036 58.328045) (end 71.12 54.542081) (width 0.2) (layer "F.Cu") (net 17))
 (segment (start 101.560425 91.479575) (end 101.560425 92.499983) (width 0.2) (layer "F.Cu") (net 17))
 (segment (start 72.86 49.06) (end 94.38 49.06) (width 0.2) (layer "F.Cu") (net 17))
 (segment (start 71.12 50.8) (end 72.86 49.06) (width 0.2) (layer "F.Cu") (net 17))
 (segment (start 86.139427 111.539427) (end 83.82 109.22) (width 0.2) (layer "F.Cu") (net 3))
 (segment (start 83.775455 93.935455) (end 79.873417 93.935455) (width 0.2) (layer "F.Cu") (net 3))
 (segment (start 87.416 111.539427) (end 86.139427 111.539427) (width 0.2) (layer "F.Cu") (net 3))
 (segment (start 83.82 109.22) (end 83.82 93.98) (width 0.2) (layer "F.Cu") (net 3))
 (segment (start 83.82 93.98) (end 83.775455 93.935455) (width 0.2) (layer "F.Cu") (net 3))
 (segment (start 79.965372 91.48741) (end 84.799852 91.48741) (width 0.2) (layer "F.Cu") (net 1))
 (segment (start 79.873417 91.395455) (end 79.965372 91.48741) (width 0.2) (layer "F.Cu") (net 1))
 (segment (start 84.799852 91.48741) (end 85.812425 92.499983) (width 0.2) (layer "F.Cu") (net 1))
 (segment (start 63.145915 71.028045) (end 58.42 75.75396) (width 0.2) (layer "F.Cu") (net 22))
 (segment (start 64.633417 71.028045) (end 63.145915 71.028045) (width 0.2) (layer "F.Cu") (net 22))
 (segment (start 55.88 83.82) (end 55.88 106.68) (width 0.2) (layer "F.Cu") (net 22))
 (segment (start 58.42 81.28) (end 55.88 83.82) (width 0.2) (layer "F.Cu") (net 22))
 (segment (start 55.88 106.68) (end 71.12 121.92) (width 0.2) (layer "F.Cu") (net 22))
 (segment (start 58.42 75.75396) (end 58.42 81.28) (width 0.2) (layer "F.Cu") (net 22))
 (segment (start 64.541462 78.74) (end 64.633417 78.648045) (width 0.2) (layer "F.Cu") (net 29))
 (segment (start 64.633417 76.108045) (end 61.563737 79.177725) (width 0.2) (layer "F.Cu") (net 27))
 (segment (start 58.82 102) (end 73.66 116.84) (width 0.2) (layer "F.Cu") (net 27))
 (segment (start 61.563737 83.674141) (end 61.617641 83.728045) (width 0.2) (layer "F.Cu") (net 27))
 (segment (start 58.82 86.525686) (end 58.82 102) (width 0.2) (layer "F.Cu") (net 27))
 (segment (start 61.563737 79.177725) (end 61.563737 83.674141) (width 0.2) (layer "F.Cu") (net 27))
 (segment (start 73.66 116.84) (end 73.66 127) (width 0.2) (layer "F.Cu") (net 27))
 (segment (start 61.617641 83.728045) (end 58.82 86.525686) (width 0.2) (layer "F.Cu") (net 27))
 (segment (start 73.66 127) (end 78.74 127) (width 0.2) (layer "F.Cu") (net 27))
 (segment (start 98.609054 48.14526) (end 98.609054 64.130823) (width 0.2) (layer "F.Cu") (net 18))
 (segment (start 98.389246 47.589246) (end 98.777157 47.977157) (width 0.2) (layer "F.Cu") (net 18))
 (segment (start 69.29876 50.08124) (end 69.29876 47.589246) (width 0.2) (layer "F.Cu") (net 18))
 (segment (start 69.29876 47.589246) (end 98.389246 47.589246) (width 0.2) (layer "F.Cu") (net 18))
 (segment (start 66.131955 53.248045) (end 69.29876 50.08124) (width 0.2) (layer "F.Cu") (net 18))
 (segment (start 64.633417 53.248045) (end 66.131955 53.248045) (width 0.2) (layer "F.Cu") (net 18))
 (segment (start 98.609054 64.130823) (end 99.009054 64.530823) (width 0.2) (layer "F.Cu") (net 18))
 (segment (start 98.777157 47.977157) (end 98.609054 48.14526) (width 0.2) (layer "F.Cu") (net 18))
 (segment (start 104.18 106.72) (end 104.18 111.539427) (width 0.2) (layer "F.Cu") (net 19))
 (segment (start 66.131955 60.868045) (end 72.197679 54.802321) (width 0.2) (layer "F.Cu") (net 19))
 (segment (start 94.972454 51.226769) (end 94.972454 92.432454) (width 0.2) (layer "F.Cu") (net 19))
 (segment (start 93.494329 49.748644) (end 94.972454 51.226769) (width 0.2) (layer "F.Cu") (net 19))
 (segment (start 94.972454 92.432454) (end 104.14 101.6) (width 0.2) (layer "F.Cu") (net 19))
 (segment (start 104.14 106.68) (end 104.18 106.72) (width 0.2) (layer "F.Cu") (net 19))
 (segment (start 104.14 101.6) (end 104.14 106.68) (width 0.2) (layer "F.Cu") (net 19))
 (segment (start 74.145671 49.748644) (end 93.494329 49.748644) (width 0.2) (layer "F.Cu") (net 19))
 (segment (start 72.197679 54.802321) (end 72.197679 51.696636) (width 0.2) (layer "F.Cu") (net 19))
 (segment (start 64.633417 60.868045) (end 66.131955 60.868045) (width 0.2) (layer "F.Cu") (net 19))
 (segment (start 72.197679 51.696636) (end 74.145671 49.748644) (width 0.2) (layer "F.Cu") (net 19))
 (segment (start 64.633417 73.568045) (end 64.541462 73.66) (width 0.2) (layer "F.Cu") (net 21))
 (segment (start 64.540279 73.661183) (end 64.633417 73.568045) (width 0.2) (layer "F.Cu") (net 21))
 (segment (start 57.326691 85.34419) (end 57.446346 85.463845) (width 0.2) (layer "F.Cu") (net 21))
 (segment (start 59.956323 82.714558) (end 57.326691 85.34419) (width 0.2) (layer "F.Cu") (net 21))
 (segment (start 57.446346 105.706346) (end 71.12 119.38) (width 0.2) (layer "F.Cu") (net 21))
 (segment (start 59.956323 77.274632) (end 59.956323 82.714558) (width 0.2) (layer "F.Cu") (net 21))
 (segment (start 63.5 73.66) (end 60.96 76.2) (width 0.2) (layer "F.Cu") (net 21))
 (segment (start 60.96 76.2) (end 60.96 76.270955) (width 0.2) (layer "F.Cu") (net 21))
 (segment (start 60.96 76.270955) (end 59.956323 77.274632) (width 0.2) (layer "F.Cu") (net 21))
 (segment (start 64.541462 73.66) (end 63.5 73.66) (width 0.2) (layer "F.Cu") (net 21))
 (segment (start 57.446346 85.463845) (end 57.446346 105.706346) (width 0.2) (layer "F.Cu") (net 21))
 (segment (start 78.74 66.04) (end 71.12 73.66) (width 0.2) (layer "F.Cu") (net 11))
 (segment (start 71.12 101.034314) (end 83.82 113.734314) (width 0.2) (layer "F.Cu") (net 11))
 (segment (start 83.82 113.734314) (end 83.82 124.46) (width 0.2) (layer "F.Cu") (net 11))
 (segment (start 79.828872 66.04) (end 78.74 66.04) (width 0.2) (layer "F.Cu") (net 11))
 (segment (start 79.873417 65.995455) (end 79.828872 66.04) (width 0.2) (layer "F.Cu") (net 11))
 (segment (start 83.82 124.46) (end 85.52305 124.46) (width 0.2) (layer "F.Cu") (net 11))
 (segment (start 71.12 73.66) (end 71.12 101.034314) (width 0.2) (layer "F.Cu") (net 11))
 (segment (start 79.917962 53.34) (end 79.873417 53.295455) (width 0.2) (layer "F.Cu") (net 16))
 (segment (start 83.82 53.34) (end 79.917962 53.34) (width 0.2) (layer "F.Cu") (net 16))
 (segment (start 84.277054 64.530823) (end 84.277054 53.797054) (width 0.2) (layer "F.Cu") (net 16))
 (segment (start 84.277054 53.797054) (end 83.82 53.34) (width 0.2) (layer "F.Cu") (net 16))
 (segment (start 93.98 127) (end 90.991471 124.011471) (width 0.2) (layer "F.Cu") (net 10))
 (segment (start 73.66 73.66) (end 78.74 68.58) (width 0.2) (layer "F.Cu") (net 10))
 (segment (start 78.74 68.58) (end 79.828872 68.58) (width 0.2) (layer "F.Cu") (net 10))
 (segment (start 90.991471 119.569891) (end 73.66 102.23842) (width 0.2) (layer "F.Cu") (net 10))
 (segment (start 95.391417 130.438924) (end 93.98 129.027507) (width 0.2) (layer "F.Cu") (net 10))
 (segment (start 79.828872 68.58) (end 79.873417 68.535455) (width 0.2) (layer "F.Cu") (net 10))
 (segment (start 90.991471 124.011471) (end 90.991471 119.569891) (width 0.2) (layer "F.Cu") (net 10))
 (segment (start 73.66 102.23842) (end 73.66 73.66) (width 0.2) (layer "F.Cu") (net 10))
 (segment (start 93.98 129.027507) (end 93.98 127) (width 0.2) (layer "F.Cu") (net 10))
 (segment (start 79.873417 73.615455) (end 83.201686 73.615455) (width 0.2) (layer "F.Cu") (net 8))
 (segment (start 83.201686 73.615455) (end 84.277054 74.690823) (width 0.2) (layer "F.Cu") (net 8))
 (segment (start 84.277054 74.690823) (end 84.277054 74.117054) (width 0.2) (layer "F.Cu") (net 8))
 (segment (start 90.17 117.261471) (end 92.427156 117.261471) (width 0.2) (layer "F.Cu") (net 9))
 (segment (start 78.74 105.831471) (end 90.17 117.261471) (width 0.2) (layer "F.Cu") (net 9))
 (segment (start 92.925328 117.759643) (end 92.925328 123.646161) (width 0.2) (layer "F.Cu") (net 9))
 (segment (start 76.2 99.06) (end 78.74 101.6) (width 0.2) (layer "F.Cu") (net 9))
 (segment (start 78.74 71.16741) (end 76.2 73.70741) (width 0.2) (layer "F.Cu") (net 9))
 (segment (start 92.925328 123.646161) (end 97.931417 128.65225) (width 0.2) (layer "F.Cu") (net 9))
 (segment (start 97.931417 128.65225) (end 97.931417 130.438924) (width 0.2) (layer "F.Cu") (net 9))
 (segment (start 76.2 73.70741) (end 76.2 99.06) (width 0.2) (layer "F.Cu") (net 9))
 (segment (start 78.69259 71.16741) (end 78.74 71.16741) (width 0.2) (layer "F.Cu") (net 9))
 (segment (start 78.74 71.16741) (end 79.781462 71.16741) (width 0.2) (layer "F.Cu") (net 9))
 (segment (start 78.74 101.6) (end 78.74 105.831471) (width 0.2) (layer "F.Cu") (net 9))
 (segment (start 92.427156 117.261471) (end 92.925328 117.759643) (width 0.2) (layer "F.Cu") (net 9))
 (segment (start 79.781462 71.16741) (end 79.873417 71.075455) (width 0.2) (layer "F.Cu") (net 9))
 (segment (start 64.541462 86.36) (end 64.633417 86.268045) (width 0.2) (layer "F.Cu") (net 30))
 (segment (start 74.639396 115.279396) (end 60.96 101.6) (width 0.2) (layer "F.Cu") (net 26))
 (segment (start 60.96 88.9) (end 61.051955 88.808045) (width 0.2) (layer "F.Cu") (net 26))
 (segment (start 61.051955 88.808045) (end 64.633417 88.808045) (width 0.2) (layer "F.Cu") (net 26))
 (segment (start 60.96 101.6) (end 60.96 88.9) (width 0.2) (layer "F.Cu") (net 26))
 (segment (start 74.639396 124.144569) (end 74.639396 115.279396) (width 0.2) (layer "F.Cu") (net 26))
 (segment (start 78.74 124.46) (end 74.954827 124.46) (width 0.2) (layer "F.Cu") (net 26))
 (segment (start 64.541462 88.9) (end 64.633417 88.808045) (width 0.2) (layer "F.Cu") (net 26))
 (segment (start 74.954827 124.46) (end 74.639396 124.144569) (width 0.2) (layer "F.Cu") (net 26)))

